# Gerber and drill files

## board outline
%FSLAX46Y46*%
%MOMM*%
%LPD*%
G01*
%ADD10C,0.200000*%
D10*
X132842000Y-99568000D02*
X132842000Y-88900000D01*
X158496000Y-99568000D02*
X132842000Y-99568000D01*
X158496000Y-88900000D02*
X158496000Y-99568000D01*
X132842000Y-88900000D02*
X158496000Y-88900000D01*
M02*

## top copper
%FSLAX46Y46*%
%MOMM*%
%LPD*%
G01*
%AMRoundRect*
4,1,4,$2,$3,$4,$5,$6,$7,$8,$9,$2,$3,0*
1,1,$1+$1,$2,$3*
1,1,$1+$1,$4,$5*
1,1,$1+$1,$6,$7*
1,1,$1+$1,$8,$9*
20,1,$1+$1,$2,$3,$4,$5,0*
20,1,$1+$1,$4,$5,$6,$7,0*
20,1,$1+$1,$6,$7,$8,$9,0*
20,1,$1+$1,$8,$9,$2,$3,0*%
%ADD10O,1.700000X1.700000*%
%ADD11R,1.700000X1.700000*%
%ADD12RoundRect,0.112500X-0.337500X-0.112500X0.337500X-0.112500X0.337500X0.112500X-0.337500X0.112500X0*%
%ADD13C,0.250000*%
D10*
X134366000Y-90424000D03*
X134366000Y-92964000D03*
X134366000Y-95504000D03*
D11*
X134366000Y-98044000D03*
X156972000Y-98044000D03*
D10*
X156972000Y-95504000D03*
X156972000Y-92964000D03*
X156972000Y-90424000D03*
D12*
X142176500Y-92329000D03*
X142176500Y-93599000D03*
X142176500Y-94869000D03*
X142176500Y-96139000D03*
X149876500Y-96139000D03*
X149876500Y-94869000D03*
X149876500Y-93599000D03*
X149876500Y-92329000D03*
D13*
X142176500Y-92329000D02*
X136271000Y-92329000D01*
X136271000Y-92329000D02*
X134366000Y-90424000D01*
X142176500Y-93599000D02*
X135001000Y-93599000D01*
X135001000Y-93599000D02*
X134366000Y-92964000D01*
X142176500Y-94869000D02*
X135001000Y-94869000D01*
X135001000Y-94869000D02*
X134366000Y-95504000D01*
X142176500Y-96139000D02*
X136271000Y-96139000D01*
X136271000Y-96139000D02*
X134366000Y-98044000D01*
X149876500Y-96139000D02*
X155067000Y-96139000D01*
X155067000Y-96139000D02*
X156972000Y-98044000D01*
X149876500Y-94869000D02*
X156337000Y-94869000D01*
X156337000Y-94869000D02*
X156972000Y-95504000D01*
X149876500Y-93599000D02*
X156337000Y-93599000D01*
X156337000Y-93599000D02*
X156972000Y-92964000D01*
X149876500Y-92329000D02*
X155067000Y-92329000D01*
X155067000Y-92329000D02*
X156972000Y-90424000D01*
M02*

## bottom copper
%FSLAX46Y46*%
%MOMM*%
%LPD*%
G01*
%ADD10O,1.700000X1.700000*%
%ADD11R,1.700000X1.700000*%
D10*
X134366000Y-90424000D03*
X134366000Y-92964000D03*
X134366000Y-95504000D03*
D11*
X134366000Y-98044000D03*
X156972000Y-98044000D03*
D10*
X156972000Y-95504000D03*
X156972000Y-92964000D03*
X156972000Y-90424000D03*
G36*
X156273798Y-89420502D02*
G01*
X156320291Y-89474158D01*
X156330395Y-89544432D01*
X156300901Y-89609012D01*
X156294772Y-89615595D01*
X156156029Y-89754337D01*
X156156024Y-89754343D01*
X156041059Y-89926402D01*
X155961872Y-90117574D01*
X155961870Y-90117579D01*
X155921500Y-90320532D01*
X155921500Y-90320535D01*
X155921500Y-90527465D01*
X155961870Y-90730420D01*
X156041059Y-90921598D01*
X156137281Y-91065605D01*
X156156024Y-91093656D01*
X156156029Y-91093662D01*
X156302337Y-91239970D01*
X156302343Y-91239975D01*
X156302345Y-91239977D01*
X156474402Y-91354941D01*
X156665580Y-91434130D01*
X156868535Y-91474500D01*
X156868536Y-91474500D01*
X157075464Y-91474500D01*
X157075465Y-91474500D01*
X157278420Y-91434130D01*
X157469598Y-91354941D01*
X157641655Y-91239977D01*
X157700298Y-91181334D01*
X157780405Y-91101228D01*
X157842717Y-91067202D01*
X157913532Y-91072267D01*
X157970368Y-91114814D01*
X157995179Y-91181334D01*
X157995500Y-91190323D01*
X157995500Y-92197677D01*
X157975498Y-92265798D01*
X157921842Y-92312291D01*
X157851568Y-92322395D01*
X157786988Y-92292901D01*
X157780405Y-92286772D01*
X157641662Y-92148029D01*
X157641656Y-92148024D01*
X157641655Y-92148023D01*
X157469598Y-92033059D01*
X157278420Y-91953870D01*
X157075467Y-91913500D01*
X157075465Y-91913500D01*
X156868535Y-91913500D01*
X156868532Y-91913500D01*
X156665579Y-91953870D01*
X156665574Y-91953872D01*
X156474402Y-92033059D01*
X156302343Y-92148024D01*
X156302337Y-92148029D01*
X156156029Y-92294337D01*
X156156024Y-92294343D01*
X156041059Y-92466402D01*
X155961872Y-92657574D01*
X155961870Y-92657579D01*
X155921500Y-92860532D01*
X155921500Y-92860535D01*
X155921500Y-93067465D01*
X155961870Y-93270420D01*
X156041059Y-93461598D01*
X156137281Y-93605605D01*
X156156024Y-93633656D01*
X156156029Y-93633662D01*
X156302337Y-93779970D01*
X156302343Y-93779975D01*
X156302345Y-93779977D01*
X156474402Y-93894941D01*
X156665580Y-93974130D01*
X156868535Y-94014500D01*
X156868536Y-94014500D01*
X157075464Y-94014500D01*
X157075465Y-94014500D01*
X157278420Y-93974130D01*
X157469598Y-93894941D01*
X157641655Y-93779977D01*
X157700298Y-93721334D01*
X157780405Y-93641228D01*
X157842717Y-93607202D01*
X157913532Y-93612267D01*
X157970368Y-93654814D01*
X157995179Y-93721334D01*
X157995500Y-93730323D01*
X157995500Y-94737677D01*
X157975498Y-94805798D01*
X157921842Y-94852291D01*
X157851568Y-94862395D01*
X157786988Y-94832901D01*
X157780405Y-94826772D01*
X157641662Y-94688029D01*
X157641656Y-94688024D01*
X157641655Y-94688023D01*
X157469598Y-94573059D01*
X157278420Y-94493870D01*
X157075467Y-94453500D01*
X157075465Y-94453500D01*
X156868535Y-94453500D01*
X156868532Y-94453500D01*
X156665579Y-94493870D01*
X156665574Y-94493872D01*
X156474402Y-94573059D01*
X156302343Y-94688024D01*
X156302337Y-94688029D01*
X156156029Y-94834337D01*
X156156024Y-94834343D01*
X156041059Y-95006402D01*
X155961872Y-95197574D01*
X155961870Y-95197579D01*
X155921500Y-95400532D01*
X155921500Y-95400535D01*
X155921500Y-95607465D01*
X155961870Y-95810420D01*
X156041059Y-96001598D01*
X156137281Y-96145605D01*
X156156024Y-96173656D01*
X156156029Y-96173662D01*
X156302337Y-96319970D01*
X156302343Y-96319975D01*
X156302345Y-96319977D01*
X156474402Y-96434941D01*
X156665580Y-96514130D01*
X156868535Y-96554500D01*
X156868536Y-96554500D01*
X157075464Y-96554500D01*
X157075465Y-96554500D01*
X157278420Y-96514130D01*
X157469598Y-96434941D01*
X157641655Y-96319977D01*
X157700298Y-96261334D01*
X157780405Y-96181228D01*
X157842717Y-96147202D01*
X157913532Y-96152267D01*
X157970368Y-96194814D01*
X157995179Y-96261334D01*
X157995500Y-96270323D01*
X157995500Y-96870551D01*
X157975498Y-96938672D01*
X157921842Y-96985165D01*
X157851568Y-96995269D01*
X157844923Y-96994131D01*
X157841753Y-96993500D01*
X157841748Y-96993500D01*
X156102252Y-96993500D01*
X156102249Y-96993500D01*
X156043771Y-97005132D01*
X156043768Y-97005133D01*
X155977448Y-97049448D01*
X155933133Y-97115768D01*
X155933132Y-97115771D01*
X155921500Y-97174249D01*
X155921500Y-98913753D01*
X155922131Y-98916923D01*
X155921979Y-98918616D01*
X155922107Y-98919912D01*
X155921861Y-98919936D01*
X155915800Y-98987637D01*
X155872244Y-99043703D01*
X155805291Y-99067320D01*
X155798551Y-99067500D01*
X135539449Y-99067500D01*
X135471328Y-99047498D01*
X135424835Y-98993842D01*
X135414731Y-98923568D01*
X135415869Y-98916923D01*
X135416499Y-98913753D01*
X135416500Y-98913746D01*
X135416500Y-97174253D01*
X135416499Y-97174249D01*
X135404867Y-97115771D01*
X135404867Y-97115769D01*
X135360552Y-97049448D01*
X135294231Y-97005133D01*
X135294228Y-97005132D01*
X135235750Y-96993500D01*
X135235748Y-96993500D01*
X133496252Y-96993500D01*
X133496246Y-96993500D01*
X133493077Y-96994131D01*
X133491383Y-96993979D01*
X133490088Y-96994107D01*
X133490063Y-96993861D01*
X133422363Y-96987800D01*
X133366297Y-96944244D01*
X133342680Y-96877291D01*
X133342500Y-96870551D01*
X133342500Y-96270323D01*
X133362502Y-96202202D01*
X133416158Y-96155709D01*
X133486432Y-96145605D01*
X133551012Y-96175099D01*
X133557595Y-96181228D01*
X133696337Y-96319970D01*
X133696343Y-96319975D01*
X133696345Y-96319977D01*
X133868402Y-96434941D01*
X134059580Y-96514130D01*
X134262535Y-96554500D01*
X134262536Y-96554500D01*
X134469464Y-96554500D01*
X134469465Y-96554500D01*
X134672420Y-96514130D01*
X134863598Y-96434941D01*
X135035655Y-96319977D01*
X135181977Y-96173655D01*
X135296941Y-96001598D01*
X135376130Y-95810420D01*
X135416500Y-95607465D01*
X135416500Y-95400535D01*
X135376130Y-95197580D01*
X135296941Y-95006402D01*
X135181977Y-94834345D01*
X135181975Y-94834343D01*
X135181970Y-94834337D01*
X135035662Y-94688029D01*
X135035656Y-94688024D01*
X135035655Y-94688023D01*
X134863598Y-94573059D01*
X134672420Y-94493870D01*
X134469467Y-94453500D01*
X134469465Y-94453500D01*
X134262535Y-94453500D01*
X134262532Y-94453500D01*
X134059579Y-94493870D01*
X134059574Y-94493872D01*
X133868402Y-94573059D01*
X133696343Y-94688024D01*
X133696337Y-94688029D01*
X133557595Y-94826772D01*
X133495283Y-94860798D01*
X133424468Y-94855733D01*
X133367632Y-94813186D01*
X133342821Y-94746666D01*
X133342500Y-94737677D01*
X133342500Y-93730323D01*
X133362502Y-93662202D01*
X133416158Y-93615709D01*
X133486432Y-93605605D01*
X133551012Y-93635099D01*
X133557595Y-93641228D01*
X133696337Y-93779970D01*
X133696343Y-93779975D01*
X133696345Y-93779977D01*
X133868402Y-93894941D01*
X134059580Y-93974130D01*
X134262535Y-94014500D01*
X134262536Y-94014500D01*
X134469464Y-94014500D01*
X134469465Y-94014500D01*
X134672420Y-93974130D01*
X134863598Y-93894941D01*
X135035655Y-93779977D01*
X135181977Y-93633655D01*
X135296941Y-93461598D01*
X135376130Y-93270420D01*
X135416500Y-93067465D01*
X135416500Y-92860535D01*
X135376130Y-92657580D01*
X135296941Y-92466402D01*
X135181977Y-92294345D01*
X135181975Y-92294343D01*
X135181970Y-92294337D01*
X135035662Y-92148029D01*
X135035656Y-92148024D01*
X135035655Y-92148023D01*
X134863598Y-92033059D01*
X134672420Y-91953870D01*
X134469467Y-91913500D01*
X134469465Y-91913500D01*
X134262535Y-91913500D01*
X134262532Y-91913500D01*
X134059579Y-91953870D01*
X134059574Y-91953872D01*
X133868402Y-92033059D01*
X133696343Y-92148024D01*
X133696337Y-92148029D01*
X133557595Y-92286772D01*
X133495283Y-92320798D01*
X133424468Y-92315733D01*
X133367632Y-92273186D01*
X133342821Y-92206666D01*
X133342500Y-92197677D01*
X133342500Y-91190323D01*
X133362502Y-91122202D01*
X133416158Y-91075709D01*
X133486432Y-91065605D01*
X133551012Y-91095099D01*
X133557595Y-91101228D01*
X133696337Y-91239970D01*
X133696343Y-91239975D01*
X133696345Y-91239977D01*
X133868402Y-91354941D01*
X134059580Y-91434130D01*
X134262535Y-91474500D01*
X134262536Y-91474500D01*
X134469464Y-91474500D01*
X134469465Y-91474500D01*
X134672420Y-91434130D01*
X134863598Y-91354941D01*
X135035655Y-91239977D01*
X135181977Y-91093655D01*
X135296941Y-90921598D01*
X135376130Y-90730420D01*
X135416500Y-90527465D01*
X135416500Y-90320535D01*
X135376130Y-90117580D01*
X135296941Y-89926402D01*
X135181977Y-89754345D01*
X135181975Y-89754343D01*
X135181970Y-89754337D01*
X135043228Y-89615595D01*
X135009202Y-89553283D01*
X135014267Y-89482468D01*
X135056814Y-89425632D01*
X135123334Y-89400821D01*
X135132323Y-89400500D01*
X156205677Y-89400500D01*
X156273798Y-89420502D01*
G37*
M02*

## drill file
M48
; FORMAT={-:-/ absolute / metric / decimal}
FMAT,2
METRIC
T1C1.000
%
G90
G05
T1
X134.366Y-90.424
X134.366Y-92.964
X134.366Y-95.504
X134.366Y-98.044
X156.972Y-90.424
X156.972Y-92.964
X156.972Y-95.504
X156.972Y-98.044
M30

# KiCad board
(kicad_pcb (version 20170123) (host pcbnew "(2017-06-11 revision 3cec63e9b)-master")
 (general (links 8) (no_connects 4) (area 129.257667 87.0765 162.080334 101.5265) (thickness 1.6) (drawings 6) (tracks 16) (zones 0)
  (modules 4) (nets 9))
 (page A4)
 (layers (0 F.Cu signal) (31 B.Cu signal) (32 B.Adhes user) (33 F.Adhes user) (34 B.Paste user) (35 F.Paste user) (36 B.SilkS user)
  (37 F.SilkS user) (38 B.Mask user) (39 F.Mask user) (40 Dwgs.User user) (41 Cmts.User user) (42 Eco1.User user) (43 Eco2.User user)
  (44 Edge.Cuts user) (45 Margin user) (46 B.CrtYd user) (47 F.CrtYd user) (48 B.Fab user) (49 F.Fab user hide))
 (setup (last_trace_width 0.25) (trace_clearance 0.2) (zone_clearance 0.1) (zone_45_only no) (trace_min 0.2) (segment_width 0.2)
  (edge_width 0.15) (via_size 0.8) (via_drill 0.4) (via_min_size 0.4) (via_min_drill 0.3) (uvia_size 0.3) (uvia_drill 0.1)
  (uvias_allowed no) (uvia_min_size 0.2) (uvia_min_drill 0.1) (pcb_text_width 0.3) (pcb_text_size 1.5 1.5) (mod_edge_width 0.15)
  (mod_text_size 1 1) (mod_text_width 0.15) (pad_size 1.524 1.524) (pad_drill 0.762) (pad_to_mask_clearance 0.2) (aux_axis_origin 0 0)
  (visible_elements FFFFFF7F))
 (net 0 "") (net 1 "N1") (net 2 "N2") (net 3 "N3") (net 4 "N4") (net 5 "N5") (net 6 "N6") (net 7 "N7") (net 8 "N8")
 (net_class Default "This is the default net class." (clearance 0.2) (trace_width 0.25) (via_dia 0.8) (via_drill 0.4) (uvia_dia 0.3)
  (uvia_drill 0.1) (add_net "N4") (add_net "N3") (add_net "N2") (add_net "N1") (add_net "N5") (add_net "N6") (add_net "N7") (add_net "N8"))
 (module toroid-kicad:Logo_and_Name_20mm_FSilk (layer B.Cu) (at 145.542 94.234)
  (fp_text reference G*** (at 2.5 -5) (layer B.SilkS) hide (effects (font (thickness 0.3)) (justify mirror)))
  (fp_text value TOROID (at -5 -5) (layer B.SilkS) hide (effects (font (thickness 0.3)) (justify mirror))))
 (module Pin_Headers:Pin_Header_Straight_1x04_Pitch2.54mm (layer F.Cu) (at 134.366 98.044 180)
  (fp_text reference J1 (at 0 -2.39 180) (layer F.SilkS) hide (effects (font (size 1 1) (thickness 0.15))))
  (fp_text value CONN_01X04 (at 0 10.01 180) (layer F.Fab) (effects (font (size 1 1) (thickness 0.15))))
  (pad 4 thru_hole oval (at 0 7.62 180) (size 1.7 1.7) (drill 1) (layers *.Cu *.Mask) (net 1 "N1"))
  (pad 3 thru_hole oval (at 0 5.08 180) (size 1.7 1.7) (drill 1) (layers *.Cu *.Mask) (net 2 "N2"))
  (pad 2 thru_hole oval (at 0 2.54 180) (size 1.7 1.7) (drill 1) (layers *.Cu *.Mask) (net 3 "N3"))
  (pad 1 thru_hole rect (at 0 0 180) (size 1.7 1.7) (drill 1) (layers *.Cu *.Mask) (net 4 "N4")))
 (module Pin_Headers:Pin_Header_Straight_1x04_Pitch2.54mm (layer F.Cu) (at 156.972 98.044 180)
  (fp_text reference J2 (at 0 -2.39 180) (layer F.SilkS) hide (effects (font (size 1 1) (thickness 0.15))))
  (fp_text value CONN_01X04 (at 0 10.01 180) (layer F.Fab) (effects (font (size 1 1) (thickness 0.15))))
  (pad 1 thru_hole rect (at 0 0 180) (size 1.7 1.7) (drill 1) (layers *.Cu *.Mask) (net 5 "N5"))
  (pad 2 thru_hole oval (at 0 2.54 180) (size 1.7 1.7) (drill 1) (layers *.Cu *.Mask) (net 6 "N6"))
  (pad 3 thru_hole oval (at 0 5.08 180) (size 1.7 1.7) (drill 1) (layers *.Cu *.Mask) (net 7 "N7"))
  (pad 4 thru_hole oval (at 0 7.62 180) (size 1.7 1.7) (drill 1) (layers *.Cu *.Mask) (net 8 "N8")))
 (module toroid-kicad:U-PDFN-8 (layer F.Cu) (at 146.05 94.234)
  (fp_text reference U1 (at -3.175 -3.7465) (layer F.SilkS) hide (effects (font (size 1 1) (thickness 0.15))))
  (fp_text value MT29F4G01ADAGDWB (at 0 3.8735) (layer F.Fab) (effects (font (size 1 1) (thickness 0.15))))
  (pad 1 smd roundrect (at -3.8735 -1.905) (size 0.9 0.45) (layers F.Cu F.Paste F.Mask) (roundrect_rratio 0.25) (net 1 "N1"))
  (pad 2 smd roundrect (at -3.8735 -0.635) (size 0.9 0.45) (layers F.Cu F.Paste F.Mask) (roundrect_rratio 0.25) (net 2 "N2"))
  (pad 3 smd roundrect (at -3.8735 0.635) (size 0.9 0.45) (layers F.Cu F.Paste F.Mask) (roundrect_rratio 0.25) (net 3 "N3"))
  (pad 4 smd roundrect (at -3.8735 1.905) (size 0.9 0.45) (layers F.Cu F.Paste F.Mask) (roundrect_rratio 0.25) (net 4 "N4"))
  (pad 5 smd roundrect (at 3.8265 1.905) (size 0.9 0.45) (layers F.Cu F.Paste F.Mask) (roundrect_rratio 0.25) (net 5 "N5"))
  (pad 6 smd roundrect (at 3.8265 0.635) (size 0.9 0.45) (layers F.Cu F.Paste F.Mask) (roundrect_rratio 0.25) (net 6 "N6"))
  (pad 7 smd roundrect (at 3.8265 -0.635) (size 0.9 0.45) (layers F.Cu F.Paste F.Mask) (roundrect_rratio 0.25) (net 7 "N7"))
  (pad 8 smd roundrect (at 3.8265 -1.905) (size 0.9 0.45) (layers F.Cu F.Paste F.Mask) (roundrect_rratio 0.25) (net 8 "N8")))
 (gr_line (start 132.842 99.568) (end 132.842 88.9) (layer Edge.Cuts) (width 0.2))
 (gr_line (start 158.496 99.568) (end 132.842 99.568) (layer Edge.Cuts) (width 0.2))
 (gr_line (start 158.496 88.9) (end 158.496 99.568) (layer Edge.Cuts) (width 0.2))
 (gr_line (start 132.842 88.9) (end 158.496 88.9) (layer Edge.Cuts) (width 0.2))
 (segment (start 142.1765 92.329) (end 136.271 92.329) (width 0.25) (layer F.Cu) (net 1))
 (segment (start 136.271 92.329) (end 134.366 90.424) (width 0.25) (layer F.Cu) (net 1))
 (segment (start 142.1765 93.599) (end 135.001 93.599) (width 0.25) (layer F.Cu) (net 2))
 (segment (start 135.001 93.599) (end 134.366 92.964) (width 0.25) (layer F.Cu) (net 2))
 (segment (start 142.1765 94.869) (end 135.001 94.869) (width 0.25) (layer F.Cu) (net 3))
 (segment (start 135.001 94.869) (end 134.366 95.504) (width 0.25) (layer F.Cu) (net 3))
 (segment (start 142.1765 96.139) (end 136.271 96.139) (width 0.25) (layer F.Cu) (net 4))
 (segment (start 136.271 96.139) (end 134.366 98.044) (width 0.25) (layer F.Cu) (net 4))
 (segment (start 149.8765 96.139) (end 155.067 96.139) (width 0.25) (layer F.Cu) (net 5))
 (segment (start 155.067 96.139) (end 156.972 98.044) (width 0.25) (layer F.Cu) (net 5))
 (segment (start 149.8765 94.869) (end 156.337 94.869) (width 0.25) (layer F.Cu) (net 6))
 (segment (start 156.337 94.869) (end 156.972 95.504) (width 0.25) (layer F.Cu) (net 6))
 (segment (start 149.8765 93.599) (end 156.337 93.599) (width 0.25) (layer F.Cu) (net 7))
 (segment (start 156.337 93.599) (end 156.972 92.964) (width 0.25) (layer F.Cu) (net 7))
 (segment (start 149.8765 92.329) (end 155.067 92.329) (width 0.25) (layer F.Cu) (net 8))
 (segment (start 155.067 92.329) (end 156.972 90.424) (width 0.25) (layer F.Cu) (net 8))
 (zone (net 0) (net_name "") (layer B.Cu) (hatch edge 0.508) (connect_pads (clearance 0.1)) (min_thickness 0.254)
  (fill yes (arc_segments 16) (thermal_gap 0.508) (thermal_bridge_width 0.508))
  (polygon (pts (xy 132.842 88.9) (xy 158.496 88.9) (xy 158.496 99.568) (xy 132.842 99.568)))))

